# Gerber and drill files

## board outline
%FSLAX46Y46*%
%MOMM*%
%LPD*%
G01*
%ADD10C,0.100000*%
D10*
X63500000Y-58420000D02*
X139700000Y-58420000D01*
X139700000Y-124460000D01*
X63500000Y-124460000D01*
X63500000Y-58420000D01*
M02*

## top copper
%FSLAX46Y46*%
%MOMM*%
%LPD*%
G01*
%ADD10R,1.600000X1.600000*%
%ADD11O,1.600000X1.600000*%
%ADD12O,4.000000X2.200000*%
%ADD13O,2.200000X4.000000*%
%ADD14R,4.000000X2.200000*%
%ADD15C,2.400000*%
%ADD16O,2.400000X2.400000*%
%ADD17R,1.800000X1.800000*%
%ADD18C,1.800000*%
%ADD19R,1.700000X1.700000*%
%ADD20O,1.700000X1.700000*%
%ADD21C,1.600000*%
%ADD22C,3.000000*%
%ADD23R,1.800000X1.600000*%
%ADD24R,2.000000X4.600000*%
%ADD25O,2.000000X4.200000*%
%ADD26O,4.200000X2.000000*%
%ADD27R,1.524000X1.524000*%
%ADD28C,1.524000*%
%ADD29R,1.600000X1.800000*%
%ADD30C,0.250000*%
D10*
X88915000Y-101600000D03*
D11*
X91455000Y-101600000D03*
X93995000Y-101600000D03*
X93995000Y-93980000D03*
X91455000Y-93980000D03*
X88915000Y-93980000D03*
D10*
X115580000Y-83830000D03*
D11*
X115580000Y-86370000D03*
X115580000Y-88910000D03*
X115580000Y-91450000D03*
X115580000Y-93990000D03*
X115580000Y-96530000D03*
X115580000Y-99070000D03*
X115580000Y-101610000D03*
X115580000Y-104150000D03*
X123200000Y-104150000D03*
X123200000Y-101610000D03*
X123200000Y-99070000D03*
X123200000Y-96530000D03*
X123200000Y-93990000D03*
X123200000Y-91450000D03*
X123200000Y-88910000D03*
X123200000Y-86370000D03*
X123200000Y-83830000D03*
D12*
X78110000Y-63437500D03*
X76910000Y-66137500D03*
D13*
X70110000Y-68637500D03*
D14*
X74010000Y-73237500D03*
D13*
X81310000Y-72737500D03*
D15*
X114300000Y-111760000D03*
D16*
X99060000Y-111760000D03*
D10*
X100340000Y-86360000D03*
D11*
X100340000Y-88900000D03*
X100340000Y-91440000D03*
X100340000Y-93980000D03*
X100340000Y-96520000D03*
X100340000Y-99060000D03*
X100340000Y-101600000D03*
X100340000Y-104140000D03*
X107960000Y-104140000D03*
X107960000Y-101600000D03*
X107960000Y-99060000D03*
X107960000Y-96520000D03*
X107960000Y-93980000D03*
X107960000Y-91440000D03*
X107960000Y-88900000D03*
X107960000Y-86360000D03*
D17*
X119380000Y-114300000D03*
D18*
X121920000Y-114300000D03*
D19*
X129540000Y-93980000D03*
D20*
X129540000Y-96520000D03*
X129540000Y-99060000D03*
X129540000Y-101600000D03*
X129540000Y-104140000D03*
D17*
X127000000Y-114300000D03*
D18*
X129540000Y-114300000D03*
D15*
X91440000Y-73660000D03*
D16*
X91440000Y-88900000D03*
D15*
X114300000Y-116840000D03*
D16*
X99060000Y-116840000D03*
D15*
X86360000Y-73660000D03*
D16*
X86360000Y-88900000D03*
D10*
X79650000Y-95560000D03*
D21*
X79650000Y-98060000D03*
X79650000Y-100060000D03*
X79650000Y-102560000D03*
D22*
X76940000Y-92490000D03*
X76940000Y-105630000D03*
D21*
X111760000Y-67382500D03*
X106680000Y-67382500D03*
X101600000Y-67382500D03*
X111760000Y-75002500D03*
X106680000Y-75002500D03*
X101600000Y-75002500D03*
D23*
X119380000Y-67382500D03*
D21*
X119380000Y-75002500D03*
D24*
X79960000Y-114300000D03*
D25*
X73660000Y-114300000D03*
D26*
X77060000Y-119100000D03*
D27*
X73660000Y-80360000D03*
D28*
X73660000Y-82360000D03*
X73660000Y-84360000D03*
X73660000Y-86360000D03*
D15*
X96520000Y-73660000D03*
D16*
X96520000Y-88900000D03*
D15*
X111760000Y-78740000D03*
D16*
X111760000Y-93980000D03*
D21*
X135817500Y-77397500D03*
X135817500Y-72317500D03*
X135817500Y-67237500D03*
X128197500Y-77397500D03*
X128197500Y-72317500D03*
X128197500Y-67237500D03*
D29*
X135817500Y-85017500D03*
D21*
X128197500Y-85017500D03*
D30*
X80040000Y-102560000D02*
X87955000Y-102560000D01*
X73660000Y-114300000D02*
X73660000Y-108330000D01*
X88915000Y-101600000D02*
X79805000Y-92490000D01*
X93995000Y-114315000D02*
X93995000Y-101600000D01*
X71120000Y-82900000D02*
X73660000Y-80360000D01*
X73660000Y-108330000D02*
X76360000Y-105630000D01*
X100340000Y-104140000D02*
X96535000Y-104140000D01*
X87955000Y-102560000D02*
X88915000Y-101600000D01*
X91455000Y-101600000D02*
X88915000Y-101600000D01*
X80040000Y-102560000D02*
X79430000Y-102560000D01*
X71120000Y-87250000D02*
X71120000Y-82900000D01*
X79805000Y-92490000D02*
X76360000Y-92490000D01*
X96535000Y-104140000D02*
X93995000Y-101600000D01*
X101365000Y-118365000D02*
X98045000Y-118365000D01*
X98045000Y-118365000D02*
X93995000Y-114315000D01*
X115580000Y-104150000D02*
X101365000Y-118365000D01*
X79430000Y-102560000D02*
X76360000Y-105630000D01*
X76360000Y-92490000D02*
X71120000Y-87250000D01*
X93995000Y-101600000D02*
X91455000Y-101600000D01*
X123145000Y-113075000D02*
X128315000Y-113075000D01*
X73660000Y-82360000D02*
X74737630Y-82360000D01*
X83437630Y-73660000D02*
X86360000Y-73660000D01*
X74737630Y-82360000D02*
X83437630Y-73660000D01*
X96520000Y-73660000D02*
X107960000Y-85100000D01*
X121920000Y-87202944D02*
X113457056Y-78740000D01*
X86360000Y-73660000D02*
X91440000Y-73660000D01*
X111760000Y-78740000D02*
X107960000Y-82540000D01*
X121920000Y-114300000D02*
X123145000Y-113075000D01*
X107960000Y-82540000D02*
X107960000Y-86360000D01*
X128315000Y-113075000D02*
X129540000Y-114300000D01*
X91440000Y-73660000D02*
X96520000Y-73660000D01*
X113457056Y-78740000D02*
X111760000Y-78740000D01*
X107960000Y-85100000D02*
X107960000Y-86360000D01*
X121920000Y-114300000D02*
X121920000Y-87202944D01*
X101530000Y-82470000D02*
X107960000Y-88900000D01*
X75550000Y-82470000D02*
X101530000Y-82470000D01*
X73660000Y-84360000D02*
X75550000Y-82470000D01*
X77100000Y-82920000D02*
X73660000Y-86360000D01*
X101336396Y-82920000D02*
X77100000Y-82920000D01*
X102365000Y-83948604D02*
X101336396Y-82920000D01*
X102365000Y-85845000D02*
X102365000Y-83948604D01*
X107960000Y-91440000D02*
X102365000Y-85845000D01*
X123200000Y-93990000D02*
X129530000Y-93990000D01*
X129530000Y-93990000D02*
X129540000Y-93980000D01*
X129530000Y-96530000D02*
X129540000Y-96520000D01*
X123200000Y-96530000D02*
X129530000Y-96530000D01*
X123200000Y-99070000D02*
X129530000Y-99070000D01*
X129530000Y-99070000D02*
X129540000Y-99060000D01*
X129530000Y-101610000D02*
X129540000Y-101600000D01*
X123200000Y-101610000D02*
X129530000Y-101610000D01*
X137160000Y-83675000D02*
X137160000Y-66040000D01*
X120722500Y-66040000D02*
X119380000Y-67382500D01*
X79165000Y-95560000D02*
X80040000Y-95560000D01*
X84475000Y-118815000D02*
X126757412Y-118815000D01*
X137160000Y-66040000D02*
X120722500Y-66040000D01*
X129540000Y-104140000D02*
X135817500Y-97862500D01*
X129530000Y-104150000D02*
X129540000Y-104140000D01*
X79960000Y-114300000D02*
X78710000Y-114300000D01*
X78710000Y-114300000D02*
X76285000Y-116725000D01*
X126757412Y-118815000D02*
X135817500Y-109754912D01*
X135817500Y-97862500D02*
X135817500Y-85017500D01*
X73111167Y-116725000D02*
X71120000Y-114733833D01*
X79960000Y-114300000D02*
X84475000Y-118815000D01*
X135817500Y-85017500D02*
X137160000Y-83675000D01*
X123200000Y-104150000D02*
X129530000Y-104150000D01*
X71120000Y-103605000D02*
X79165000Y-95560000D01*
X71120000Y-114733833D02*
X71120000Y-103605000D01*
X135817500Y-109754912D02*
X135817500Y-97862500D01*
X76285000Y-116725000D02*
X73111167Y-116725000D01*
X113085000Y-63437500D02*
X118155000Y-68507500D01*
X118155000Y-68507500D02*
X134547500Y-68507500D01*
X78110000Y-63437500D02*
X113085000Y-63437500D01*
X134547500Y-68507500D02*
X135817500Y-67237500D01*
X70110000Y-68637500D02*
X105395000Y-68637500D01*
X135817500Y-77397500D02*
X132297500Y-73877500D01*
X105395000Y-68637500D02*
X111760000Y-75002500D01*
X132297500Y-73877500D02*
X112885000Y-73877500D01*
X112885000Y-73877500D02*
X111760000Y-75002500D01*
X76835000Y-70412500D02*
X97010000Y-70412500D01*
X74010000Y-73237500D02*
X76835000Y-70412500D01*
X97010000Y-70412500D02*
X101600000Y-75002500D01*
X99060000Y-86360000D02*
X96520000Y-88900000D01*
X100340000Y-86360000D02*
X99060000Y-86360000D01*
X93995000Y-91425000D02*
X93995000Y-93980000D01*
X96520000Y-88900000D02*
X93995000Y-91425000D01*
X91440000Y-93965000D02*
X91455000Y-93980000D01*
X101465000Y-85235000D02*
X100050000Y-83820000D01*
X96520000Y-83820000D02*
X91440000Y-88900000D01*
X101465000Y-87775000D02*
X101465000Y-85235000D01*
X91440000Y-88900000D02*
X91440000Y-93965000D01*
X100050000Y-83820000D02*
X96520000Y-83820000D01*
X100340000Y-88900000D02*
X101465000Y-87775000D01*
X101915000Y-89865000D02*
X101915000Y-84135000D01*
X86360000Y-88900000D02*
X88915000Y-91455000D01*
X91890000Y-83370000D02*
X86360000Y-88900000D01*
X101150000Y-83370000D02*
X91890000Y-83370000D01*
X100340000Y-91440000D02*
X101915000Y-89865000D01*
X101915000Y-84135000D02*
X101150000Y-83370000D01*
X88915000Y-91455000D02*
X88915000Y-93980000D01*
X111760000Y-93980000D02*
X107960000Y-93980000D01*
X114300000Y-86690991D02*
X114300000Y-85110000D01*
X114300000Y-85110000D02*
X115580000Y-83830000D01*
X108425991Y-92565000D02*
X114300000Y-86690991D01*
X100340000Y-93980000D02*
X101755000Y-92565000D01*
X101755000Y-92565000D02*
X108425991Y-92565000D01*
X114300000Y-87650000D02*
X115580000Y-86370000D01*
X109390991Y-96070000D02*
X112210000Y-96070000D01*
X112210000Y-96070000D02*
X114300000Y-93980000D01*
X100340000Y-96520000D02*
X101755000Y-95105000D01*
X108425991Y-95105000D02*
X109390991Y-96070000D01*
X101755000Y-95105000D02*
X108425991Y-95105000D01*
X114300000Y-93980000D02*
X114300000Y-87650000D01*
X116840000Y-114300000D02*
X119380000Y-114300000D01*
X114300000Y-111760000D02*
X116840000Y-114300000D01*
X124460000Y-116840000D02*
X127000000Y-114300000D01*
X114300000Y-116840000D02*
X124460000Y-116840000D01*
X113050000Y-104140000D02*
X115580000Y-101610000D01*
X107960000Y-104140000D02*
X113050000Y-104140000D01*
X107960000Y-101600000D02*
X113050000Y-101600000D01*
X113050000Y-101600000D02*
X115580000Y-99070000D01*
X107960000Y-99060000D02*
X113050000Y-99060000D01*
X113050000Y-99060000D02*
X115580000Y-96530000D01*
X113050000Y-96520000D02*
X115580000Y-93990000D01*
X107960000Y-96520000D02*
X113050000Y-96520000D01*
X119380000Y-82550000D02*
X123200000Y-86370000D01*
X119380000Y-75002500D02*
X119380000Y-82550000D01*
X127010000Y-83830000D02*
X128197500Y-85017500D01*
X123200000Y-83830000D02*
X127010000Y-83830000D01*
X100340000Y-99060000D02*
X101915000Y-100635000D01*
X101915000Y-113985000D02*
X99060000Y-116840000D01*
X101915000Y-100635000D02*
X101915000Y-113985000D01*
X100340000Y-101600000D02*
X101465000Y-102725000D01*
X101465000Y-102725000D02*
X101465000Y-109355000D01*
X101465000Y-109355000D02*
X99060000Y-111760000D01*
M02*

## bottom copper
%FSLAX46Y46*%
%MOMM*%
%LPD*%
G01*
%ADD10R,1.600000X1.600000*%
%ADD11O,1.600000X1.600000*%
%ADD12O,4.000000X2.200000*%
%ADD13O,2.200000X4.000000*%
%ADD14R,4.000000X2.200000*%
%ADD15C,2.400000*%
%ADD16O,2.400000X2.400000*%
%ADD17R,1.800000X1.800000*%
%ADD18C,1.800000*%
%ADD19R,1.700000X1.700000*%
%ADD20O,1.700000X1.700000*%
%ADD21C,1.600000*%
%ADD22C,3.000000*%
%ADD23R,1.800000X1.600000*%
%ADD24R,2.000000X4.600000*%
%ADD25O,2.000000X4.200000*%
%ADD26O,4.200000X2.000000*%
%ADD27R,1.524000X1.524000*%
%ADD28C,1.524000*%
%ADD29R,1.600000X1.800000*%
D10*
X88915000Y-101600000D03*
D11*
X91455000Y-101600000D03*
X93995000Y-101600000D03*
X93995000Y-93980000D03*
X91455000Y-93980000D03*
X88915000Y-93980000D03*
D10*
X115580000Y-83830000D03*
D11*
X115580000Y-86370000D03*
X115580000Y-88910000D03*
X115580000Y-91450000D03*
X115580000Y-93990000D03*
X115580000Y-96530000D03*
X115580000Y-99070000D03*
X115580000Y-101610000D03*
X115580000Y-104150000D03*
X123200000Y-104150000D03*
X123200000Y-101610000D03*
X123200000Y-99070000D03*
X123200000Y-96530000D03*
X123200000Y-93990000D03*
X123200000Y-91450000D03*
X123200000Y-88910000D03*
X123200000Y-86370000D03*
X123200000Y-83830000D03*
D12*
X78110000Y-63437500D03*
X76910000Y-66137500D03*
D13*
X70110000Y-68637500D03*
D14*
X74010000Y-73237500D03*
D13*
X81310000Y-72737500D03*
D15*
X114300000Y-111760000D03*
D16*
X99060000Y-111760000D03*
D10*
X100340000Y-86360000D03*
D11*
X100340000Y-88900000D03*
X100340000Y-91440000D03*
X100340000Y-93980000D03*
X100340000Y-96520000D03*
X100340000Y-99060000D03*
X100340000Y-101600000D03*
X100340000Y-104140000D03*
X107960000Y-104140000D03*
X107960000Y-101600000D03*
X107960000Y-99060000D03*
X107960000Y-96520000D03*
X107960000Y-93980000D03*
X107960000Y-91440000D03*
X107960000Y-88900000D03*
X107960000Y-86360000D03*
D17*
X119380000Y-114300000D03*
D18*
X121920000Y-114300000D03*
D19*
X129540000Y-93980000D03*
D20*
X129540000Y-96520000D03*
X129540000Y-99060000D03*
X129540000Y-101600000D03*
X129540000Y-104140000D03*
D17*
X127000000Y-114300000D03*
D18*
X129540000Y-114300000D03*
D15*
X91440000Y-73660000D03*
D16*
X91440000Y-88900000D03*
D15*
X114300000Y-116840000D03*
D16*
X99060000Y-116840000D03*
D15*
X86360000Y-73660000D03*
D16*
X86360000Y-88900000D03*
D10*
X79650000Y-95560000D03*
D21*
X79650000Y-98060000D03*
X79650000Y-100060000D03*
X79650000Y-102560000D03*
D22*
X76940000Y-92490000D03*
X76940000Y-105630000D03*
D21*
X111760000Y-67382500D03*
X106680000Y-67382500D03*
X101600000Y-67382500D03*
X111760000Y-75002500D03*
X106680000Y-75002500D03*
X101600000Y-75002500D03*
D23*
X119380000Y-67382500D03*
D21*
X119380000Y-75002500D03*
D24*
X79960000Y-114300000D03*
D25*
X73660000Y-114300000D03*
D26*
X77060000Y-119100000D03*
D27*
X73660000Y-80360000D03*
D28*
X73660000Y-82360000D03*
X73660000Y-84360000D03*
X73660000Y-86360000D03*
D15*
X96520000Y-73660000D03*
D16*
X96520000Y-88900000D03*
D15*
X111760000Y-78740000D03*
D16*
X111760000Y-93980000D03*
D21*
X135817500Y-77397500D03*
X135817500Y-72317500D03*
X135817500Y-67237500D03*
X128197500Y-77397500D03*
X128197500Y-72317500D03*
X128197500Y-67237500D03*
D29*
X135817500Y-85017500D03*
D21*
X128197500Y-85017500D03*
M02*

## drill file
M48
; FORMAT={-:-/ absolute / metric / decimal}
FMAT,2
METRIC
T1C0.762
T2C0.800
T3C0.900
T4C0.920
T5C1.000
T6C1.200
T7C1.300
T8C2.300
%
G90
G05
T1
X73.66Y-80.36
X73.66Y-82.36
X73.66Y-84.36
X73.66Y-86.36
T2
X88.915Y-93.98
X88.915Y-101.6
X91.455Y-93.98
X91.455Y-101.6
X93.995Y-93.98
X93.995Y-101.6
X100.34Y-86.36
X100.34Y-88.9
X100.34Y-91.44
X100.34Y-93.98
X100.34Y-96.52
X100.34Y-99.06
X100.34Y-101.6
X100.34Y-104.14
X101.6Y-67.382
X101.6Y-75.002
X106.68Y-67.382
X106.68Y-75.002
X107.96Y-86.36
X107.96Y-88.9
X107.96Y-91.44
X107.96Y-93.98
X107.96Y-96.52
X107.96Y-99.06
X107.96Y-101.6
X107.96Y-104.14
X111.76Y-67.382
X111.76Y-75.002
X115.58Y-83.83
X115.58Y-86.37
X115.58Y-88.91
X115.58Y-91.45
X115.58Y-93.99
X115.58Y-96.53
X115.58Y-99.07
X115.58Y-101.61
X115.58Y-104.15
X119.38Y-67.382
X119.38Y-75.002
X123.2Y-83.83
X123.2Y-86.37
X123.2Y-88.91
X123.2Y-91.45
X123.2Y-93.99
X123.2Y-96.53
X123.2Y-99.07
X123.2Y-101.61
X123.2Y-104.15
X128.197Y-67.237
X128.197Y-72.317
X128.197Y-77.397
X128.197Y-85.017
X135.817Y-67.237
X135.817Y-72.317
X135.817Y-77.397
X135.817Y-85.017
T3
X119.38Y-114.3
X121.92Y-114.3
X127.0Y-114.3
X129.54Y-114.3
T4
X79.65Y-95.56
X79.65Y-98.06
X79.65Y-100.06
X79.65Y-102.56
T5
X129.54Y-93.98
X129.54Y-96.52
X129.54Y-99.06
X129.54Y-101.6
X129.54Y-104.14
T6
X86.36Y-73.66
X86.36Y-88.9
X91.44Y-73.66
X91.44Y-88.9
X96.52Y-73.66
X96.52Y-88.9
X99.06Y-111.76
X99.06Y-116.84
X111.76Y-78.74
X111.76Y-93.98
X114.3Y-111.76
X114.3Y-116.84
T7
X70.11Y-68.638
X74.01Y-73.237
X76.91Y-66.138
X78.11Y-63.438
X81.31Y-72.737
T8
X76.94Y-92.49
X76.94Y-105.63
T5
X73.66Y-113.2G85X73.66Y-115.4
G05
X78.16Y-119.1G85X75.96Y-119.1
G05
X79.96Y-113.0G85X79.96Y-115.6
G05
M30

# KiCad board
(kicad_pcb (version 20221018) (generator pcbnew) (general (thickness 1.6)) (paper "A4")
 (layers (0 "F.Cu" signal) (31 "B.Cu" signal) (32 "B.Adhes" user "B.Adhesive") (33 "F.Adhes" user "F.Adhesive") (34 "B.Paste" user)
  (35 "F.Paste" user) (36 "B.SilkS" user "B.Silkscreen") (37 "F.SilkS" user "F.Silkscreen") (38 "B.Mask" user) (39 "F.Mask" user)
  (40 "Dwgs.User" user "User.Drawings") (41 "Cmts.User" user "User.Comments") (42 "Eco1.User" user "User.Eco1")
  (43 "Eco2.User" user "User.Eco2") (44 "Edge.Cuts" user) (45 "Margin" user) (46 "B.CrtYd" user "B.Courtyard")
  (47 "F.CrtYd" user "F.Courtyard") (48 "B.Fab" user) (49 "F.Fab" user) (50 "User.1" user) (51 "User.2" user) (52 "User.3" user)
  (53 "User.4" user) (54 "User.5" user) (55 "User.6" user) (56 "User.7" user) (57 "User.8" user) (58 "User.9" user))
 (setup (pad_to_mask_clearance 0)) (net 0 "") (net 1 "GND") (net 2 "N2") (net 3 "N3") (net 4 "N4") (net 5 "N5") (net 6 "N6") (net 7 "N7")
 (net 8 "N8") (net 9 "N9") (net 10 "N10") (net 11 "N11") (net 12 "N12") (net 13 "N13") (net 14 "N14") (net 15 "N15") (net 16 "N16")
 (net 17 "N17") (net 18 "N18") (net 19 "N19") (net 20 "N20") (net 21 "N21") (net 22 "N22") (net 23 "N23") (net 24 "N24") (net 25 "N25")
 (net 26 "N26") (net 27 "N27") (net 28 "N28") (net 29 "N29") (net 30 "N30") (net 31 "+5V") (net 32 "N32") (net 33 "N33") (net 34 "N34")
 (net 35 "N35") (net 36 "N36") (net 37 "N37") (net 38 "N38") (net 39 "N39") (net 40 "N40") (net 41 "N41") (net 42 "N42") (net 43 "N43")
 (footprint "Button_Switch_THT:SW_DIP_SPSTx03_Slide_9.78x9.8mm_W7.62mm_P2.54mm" (layer "F.Cu") (at 88.915 101.6 90)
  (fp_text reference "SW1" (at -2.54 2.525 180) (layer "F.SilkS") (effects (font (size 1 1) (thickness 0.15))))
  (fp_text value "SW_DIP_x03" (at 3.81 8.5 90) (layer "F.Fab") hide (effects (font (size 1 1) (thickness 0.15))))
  (pad "1" thru_hole rect (at 0 0 90) (size 1.6 1.6) (drill 0.8) (layers "*.Cu" "*.Mask") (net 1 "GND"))
  (pad "2" thru_hole oval (at 0 2.54 90) (size 1.6 1.6) (drill 0.8) (layers "*.Cu" "*.Mask") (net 1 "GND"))
  (pad "3" thru_hole oval (at 0 5.08 90) (size 1.6 1.6) (drill 0.8) (layers "*.Cu" "*.Mask") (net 1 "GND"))
  (pad "4" thru_hole oval (at 7.62 5.08 90) (size 1.6 1.6) (drill 0.8) (layers "*.Cu" "*.Mask") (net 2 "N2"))
  (pad "5" thru_hole oval (at 7.62 2.54 90) (size 1.6 1.6) (drill 0.8) (layers "*.Cu" "*.Mask") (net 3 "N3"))
  (pad "6" thru_hole oval (at 7.62 0 90) (size 1.6 1.6) (drill 0.8) (layers "*.Cu" "*.Mask") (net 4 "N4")))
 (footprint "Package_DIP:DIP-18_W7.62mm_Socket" (layer "F.Cu") (at 115.58 83.83)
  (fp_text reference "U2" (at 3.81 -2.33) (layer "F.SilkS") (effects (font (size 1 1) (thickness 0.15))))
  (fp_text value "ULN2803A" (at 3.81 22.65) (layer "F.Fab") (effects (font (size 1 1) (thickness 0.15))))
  (pad "1" thru_hole rect (at 0 0) (size 1.6 1.6) (drill 0.8) (layers "*.Cu" "*.Mask") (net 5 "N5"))
  (pad "2" thru_hole oval (at 0 2.54) (size 1.6 1.6) (drill 0.8) (layers "*.Cu" "*.Mask") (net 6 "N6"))
  (pad "3" thru_hole oval (at 0 5.08) (size 1.6 1.6) (drill 0.8) (layers "*.Cu" "*.Mask") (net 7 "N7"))
  (pad "4" thru_hole oval (at 0 7.62) (size 1.6 1.6) (drill 0.8) (layers "*.Cu" "*.Mask") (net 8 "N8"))
  (pad "5" thru_hole oval (at 0 10.16) (size 1.6 1.6) (drill 0.8) (layers "*.Cu" "*.Mask") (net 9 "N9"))
  (pad "6" thru_hole oval (at 0 12.7) (size 1.6 1.6) (drill 0.8) (layers "*.Cu" "*.Mask") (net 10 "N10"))
  (pad "7" thru_hole oval (at 0 15.24) (size 1.6 1.6) (drill 0.8) (layers "*.Cu" "*.Mask") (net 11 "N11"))
  (pad "8" thru_hole oval (at 0 17.78) (size 1.6 1.6) (drill 0.8) (layers "*.Cu" "*.Mask") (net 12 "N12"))
  (pad "9" thru_hole oval (at 0 20.32) (size 1.6 1.6) (drill 0.8) (layers "*.Cu" "*.Mask") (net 1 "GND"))
  (pad "10" thru_hole oval (at 7.62 20.32) (size 1.6 1.6) (drill 0.8) (layers "*.Cu" "*.Mask") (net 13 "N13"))
  (pad "11" thru_hole oval (at 7.62 17.78) (size 1.6 1.6) (drill 0.8) (layers "*.Cu" "*.Mask") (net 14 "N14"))
  (pad "12" thru_hole oval (at 7.62 15.24) (size 1.6 1.6) (drill 0.8) (layers "*.Cu" "*.Mask") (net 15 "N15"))
  (pad "13" thru_hole oval (at 7.62 12.7) (size 1.6 1.6) (drill 0.8) (layers "*.Cu" "*.Mask") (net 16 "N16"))
  (pad "14" thru_hole oval (at 7.62 10.16) (size 1.6 1.6) (drill 0.8) (layers "*.Cu" "*.Mask") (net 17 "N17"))
  (pad "15" thru_hole oval (at 7.62 7.62) (size 1.6 1.6) (drill 0.8) (layers "*.Cu" "*.Mask") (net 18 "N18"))
  (pad "16" thru_hole oval (at 7.62 5.08) (size 1.6 1.6) (drill 0.8) (layers "*.Cu" "*.Mask") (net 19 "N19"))
  (pad "17" thru_hole oval (at 7.62 2.54) (size 1.6 1.6) (drill 0.8) (layers "*.Cu" "*.Mask") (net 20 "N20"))
  (pad "18" thru_hole oval (at 7.62 0) (size 1.6 1.6) (drill 0.8) (layers "*.Cu" "*.Mask") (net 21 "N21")))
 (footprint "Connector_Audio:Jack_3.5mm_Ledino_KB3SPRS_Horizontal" (layer "F.Cu") (at 74.01 73.2375)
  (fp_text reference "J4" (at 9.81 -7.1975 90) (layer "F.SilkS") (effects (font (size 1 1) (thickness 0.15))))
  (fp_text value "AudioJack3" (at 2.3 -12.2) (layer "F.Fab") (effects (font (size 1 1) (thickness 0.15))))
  (pad "R" thru_hole oval (at 4.1 -9.8) (size 4 2.2) (drill 1.3) (layers "*.Cu" "*.Mask") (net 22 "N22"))
  (pad "RN" thru_hole oval (at 2.9 -7.1) (size 4 2.2) (drill 1.3) (layers "*.Cu" "*.Mask"))
  (pad "S" thru_hole oval (at -3.9 -4.6) (size 2.2 4) (drill 1.3) (layers "*.Cu" "*.Mask") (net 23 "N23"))
  (pad "T" thru_hole rect (at 0 0) (size 4 2.2) (drill 1.3) (layers "*.Cu" "*.Mask") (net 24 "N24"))
  (pad "TN" thru_hole oval (at 7.3 -0.5 90) (size 4 2.2) (drill 1.3) (layers "*.Cu" "*.Mask")))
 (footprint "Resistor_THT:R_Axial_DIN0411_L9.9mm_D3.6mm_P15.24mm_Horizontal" (layer "F.Cu") (at 114.3 111.76 180)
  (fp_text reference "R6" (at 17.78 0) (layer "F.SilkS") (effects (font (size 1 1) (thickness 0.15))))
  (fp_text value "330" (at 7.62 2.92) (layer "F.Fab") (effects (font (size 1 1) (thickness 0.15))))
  (pad "1" thru_hole circle (at 0 0 180) (size 2.4 2.4) (drill 1.2) (layers "*.Cu" "*.Mask") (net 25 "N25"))
  (pad "2" thru_hole oval (at 15.24 0 180) (size 2.4 2.4) (drill 1.2) (layers "*.Cu" "*.Mask") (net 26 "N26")))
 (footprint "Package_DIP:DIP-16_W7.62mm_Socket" (layer "F.Cu") (at 100.34 86.36)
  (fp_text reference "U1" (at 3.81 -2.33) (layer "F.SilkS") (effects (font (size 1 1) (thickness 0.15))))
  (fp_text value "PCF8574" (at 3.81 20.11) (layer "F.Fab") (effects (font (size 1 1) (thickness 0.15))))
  (pad "1" thru_hole rect (at 0 0) (size 1.6 1.6) (drill 0.8) (layers "*.Cu" "*.Mask") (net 2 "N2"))
  (pad "2" thru_hole oval (at 0 2.54) (size 1.6 1.6) (drill 0.8) (layers "*.Cu" "*.Mask") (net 3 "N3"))
  (pad "3" thru_hole oval (at 0 5.08) (size 1.6 1.6) (drill 0.8) (layers "*.Cu" "*.Mask") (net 4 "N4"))
  (pad "4" thru_hole oval (at 0 7.62) (size 1.6 1.6) (drill 0.8) (layers "*.Cu" "*.Mask") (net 5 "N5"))
  (pad "5" thru_hole oval (at 0 10.16) (size 1.6 1.6) (drill 0.8) (layers "*.Cu" "*.Mask") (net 6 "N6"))
  (pad "6" thru_hole oval (at 0 12.7) (size 1.6 1.6) (drill 0.8) (layers "*.Cu" "*.Mask") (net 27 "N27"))
  (pad "7" thru_hole oval (at 0 15.24) (size 1.6 1.6) (drill 0.8) (layers "*.Cu" "*.Mask") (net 26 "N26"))
  (pad "8" thru_hole oval (at 0 17.78) (size 1.6 1.6) (drill 0.8) (layers "*.Cu" "*.Mask") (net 1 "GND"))
  (pad "9" thru_hole oval (at 7.62 17.78) (size 1.6 1.6) (drill 0.8) (layers "*.Cu" "*.Mask") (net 12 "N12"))
  (pad "10" thru_hole oval (at 7.62 15.24) (size 1.6 1.6) (drill 0.8) (layers "*.Cu" "*.Mask") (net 11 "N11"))
  (pad "11" thru_hole oval (at 7.62 12.7) (size 1.6 1.6) (drill 0.8) (layers "*.Cu" "*.Mask") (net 10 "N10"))
  (pad "12" thru_hole oval (at 7.62 10.16) (size 1.6 1.6) (drill 0.8) (layers "*.Cu" "*.Mask") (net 9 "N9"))
  (pad "13" thru_hole oval (at 7.62 7.62) (size 1.6 1.6) (drill 0.8) (layers "*.Cu" "*.Mask") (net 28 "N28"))
  (pad "14" thru_hole oval (at 7.62 5.08) (size 1.6 1.6) (drill 0.8) (layers "*.Cu" "*.Mask") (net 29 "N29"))
  (pad "15" thru_hole oval (at 7.62 2.54) (size 1.6 1.6) (drill 0.8) (layers "*.Cu" "*.Mask") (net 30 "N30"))
  (pad "16" thru_hole oval (at 7.62 0) (size 1.6 1.6) (drill 0.8) (layers "*.Cu" "*.Mask") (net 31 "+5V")))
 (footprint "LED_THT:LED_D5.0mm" (layer "F.Cu") (at 119.38 114.3)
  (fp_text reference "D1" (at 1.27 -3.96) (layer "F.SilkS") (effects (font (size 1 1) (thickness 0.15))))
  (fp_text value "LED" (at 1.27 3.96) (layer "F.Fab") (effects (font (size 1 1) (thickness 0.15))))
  (pad "1" thru_hole rect (at 0 0) (size 1.8 1.8) (drill 0.9) (layers "*.Cu" "*.Mask") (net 25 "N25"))
  (pad "2" thru_hole circle (at 2.54 0) (size 1.8 1.8) (drill 0.9) (layers "*.Cu" "*.Mask") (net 31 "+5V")))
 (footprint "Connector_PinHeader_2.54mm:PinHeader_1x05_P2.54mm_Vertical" (layer "F.Cu") (at 129.54 93.98)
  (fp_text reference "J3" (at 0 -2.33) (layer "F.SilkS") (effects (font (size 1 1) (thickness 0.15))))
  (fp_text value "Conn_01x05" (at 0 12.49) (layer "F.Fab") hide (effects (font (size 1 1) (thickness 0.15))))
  (pad "1" thru_hole rect (at 0 0) (size 1.7 1.7) (drill 1) (layers "*.Cu" "*.Mask") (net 17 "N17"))
  (pad "2" thru_hole oval (at 0 2.54) (size 1.7 1.7) (drill 1) (layers "*.Cu" "*.Mask") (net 16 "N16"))
  (pad "3" thru_hole oval (at 0 5.08) (size 1.7 1.7) (drill 1) (layers "*.Cu" "*.Mask") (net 15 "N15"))
  (pad "4" thru_hole oval (at 0 7.62) (size 1.7 1.7) (drill 1) (layers "*.Cu" "*.Mask") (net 14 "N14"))
  (pad "5" thru_hole oval (at 0 10.16) (size 1.7 1.7) (drill 1) (layers "*.Cu" "*.Mask") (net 13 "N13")))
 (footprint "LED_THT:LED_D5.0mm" (layer "F.Cu") (at 127 114.3)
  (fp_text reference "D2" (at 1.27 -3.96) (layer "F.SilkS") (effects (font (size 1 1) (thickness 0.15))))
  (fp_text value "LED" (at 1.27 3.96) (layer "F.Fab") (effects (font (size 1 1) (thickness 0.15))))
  (pad "1" thru_hole rect (at 0 0) (size 1.8 1.8) (drill 0.9) (layers "*.Cu" "*.Mask") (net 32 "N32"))
  (pad "2" thru_hole circle (at 2.54 0) (size 1.8 1.8) (drill 0.9) (layers "*.Cu" "*.Mask") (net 31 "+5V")))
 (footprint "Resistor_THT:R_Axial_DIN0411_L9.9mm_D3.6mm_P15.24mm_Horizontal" (layer "F.Cu") (at 91.44 73.66 -90)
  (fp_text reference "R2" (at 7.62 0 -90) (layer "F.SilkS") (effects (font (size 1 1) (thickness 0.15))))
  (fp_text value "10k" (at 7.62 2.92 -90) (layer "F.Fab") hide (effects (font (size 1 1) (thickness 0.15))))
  (pad "1" thru_hole circle (at 0 0 270) (size 2.4 2.4) (drill 1.2) (layers "*.Cu" "*.Mask") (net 31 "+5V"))
  (pad "2" thru_hole oval (at 15.24 0 270) (size 2.4 2.4) (drill 1.2) (layers "*.Cu" "*.Mask") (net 3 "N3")))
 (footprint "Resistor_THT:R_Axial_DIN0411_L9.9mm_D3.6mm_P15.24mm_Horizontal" (layer "F.Cu") (at 114.3 116.84 180)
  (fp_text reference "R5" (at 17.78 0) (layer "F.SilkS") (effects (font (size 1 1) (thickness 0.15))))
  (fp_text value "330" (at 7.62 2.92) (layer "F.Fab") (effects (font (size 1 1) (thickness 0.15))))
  (pad "1" thru_hole circle (at 0 0 180) (size 2.4 2.4) (drill 1.2) (layers "*.Cu" "*.Mask") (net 32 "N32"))
  (pad "2" thru_hole oval (at 15.24 0 180) (size 2.4 2.4) (drill 1.2) (layers "*.Cu" "*.Mask") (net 27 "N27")))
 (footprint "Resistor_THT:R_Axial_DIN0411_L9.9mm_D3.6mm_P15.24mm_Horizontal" (layer "F.Cu") (at 86.36 73.66 -90)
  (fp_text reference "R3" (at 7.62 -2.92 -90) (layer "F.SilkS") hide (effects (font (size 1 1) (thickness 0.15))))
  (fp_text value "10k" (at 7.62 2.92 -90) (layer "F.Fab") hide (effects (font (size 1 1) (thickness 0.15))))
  (pad "1" thru_hole circle (at 0 0 270) (size 2.4 2.4) (drill 1.2) (layers "*.Cu" "*.Mask") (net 31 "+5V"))
  (pad "2" thru_hole oval (at 15.24 0 270) (size 2.4 2.4) (drill 1.2) (layers "*.Cu" "*.Mask") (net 4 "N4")))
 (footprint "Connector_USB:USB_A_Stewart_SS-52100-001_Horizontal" (layer "F.Cu") (at 79.65 95.56 -90)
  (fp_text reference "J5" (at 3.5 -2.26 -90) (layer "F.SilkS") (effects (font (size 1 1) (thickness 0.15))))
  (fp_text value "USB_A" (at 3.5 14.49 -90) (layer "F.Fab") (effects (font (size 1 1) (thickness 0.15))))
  (pad "1" thru_hole rect (at 0 0 270) (size 1.6 1.6) (drill 0.92) (layers "*.Cu" "*.Mask") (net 13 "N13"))
  (pad "2" thru_hole circle (at 2.5 0 270) (size 1.6 1.6) (drill 0.92) (layers "*.Cu" "*.Mask") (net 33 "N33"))
  (pad "3" thru_hole circle (at 4.5 0 270) (size 1.6 1.6) (drill 0.92) (layers "*.Cu" "*.Mask") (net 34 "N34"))
  (pad "4" thru_hole circle (at 7 0 270) (size 1.6 1.6) (drill 0.92) (layers "*.Cu" "*.Mask") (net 1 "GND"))
  (pad "5" thru_hole circle (at -3.07 2.71 270) (size 3 3) (drill 2.3) (layers "*.Cu" "*.Mask") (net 1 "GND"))
  (pad "5" thru_hole circle (at 10.07 2.71 270) (size 3 3) (drill 2.3) (layers "*.Cu" "*.Mask") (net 1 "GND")))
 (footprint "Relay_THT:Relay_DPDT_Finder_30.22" (layer "F.Cu") (at 119.38 67.3825 180)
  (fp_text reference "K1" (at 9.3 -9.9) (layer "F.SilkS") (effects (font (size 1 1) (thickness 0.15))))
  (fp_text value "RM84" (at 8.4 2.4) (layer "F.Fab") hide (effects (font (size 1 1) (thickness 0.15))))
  (pad "11" thru_hole circle (at 7.62 0 270) (size 1.6 1.6) (drill 0.8) (layers "*.Cu" "*.Mask") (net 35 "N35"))
  (pad "12" thru_hole circle (at 12.7 0 270) (size 1.6 1.6) (drill 0.8) (layers "*.Cu" "*.Mask") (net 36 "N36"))
  (pad "14" thru_hole circle (at 17.78 0 270) (size 1.6 1.6) (drill 0.8) (layers "*.Cu" "*.Mask") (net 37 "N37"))
  (pad "21" thru_hole circle (at 7.62 -7.62 270) (size 1.6 1.6) (drill 0.8) (layers "*.Cu" "*.Mask") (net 23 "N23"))
  (pad "22" thru_hole circle (at 12.7 -7.62 270) (size 1.6 1.6) (drill 0.8) (layers "*.Cu" "*.Mask") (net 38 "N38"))
  (pad "24" thru_hole circle (at 17.78 -7.62) (size 1.6 1.6) (drill 0.8) (layers "*.Cu" "*.Mask") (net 24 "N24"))
  (pad "A1" thru_hole rect (at 0 0 270) (size 1.6 1.8) (drill 0.8) (layers "*.Cu" "*.Mask") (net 13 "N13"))
  (pad "A2" thru_hole circle (at 0 -7.62 270) (size 1.6 1.6) (drill 0.8) (layers "*.Cu" "*.Mask") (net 20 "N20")))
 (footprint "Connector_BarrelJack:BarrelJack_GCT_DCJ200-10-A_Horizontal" (layer "F.Cu") (at 79.96 114.3 -90)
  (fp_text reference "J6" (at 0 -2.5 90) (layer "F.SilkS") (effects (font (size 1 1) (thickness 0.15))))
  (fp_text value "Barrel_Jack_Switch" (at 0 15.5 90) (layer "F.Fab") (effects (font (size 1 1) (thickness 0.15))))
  (pad "1" thru_hole rect (at 0 0 270) (size 4.6 2) (drill oval 3.6 1) (layers "*.Cu" "*.Mask") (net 13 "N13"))
  (pad "2" thru_hole oval (at 0 6.3 270) (size 4.2 2) (drill oval 3.2 1) (layers "*.Cu" "*.Mask") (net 1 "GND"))
  (pad "3" thru_hole oval (at 4.8 2.9 270) (size 2 4.2) (drill oval 1 3.2) (layers "*.Cu" "*.Mask") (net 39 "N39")))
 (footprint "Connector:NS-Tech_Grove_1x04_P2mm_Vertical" (layer "F.Cu") (at 73.66 80.36)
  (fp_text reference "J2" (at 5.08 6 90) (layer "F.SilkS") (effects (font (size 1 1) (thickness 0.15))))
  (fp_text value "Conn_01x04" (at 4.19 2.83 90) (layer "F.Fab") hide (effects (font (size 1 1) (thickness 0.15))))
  (pad "1" thru_hole rect (at 0 0) (size 1.524 1.524) (drill 0.762) (layers "*.Cu" "*.Mask") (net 1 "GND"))
  (pad "2" thru_hole circle (at 0 2) (size 1.524 1.524) (drill 0.762) (layers "*.Cu" "*.Mask") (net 31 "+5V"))
  (pad "3" thru_hole circle (at 0 4) (size 1.524 1.524) (drill 0.762) (layers "*.Cu" "*.Mask") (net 30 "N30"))
  (pad "4" thru_hole circle (at 0 6) (size 1.524 1.524) (drill 0.762) (layers "*.Cu" "*.Mask") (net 29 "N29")))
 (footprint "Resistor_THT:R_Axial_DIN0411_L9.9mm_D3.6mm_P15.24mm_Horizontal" (layer "F.Cu") (at 96.52 73.66 -90)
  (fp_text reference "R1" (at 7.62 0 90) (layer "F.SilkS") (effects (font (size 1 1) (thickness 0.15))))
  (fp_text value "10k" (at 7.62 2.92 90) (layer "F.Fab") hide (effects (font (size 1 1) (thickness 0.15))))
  (pad "1" thru_hole circle (at 0 0 270) (size 2.4 2.4) (drill 1.2) (layers "*.Cu" "*.Mask") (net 31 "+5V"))
  (pad "2" thru_hole oval (at 15.24 0 270) (size 2.4 2.4) (drill 1.2) (layers "*.Cu" "*.Mask") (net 2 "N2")))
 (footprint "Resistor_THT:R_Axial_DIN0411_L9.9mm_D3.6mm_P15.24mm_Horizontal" (layer "F.Cu") (at 111.76 78.74 -90)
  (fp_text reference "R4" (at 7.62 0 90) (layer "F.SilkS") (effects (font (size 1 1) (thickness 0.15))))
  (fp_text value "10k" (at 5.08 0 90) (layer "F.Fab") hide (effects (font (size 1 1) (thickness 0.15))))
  (pad "1" thru_hole circle (at 0 0 270) (size 2.4 2.4) (drill 1.2) (layers "*.Cu" "*.Mask") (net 31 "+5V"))
  (pad "2" thru_hole oval (at 15.24 0 270) (size 2.4 2.4) (drill 1.2) (layers "*.Cu" "*.Mask") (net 28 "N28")))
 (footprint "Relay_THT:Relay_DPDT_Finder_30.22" (layer "F.Cu") (at 135.8175 85.0175 90)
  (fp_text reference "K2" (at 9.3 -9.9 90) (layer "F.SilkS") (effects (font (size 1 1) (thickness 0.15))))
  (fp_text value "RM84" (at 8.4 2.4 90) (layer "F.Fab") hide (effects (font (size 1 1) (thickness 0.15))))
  (pad "11" thru_hole circle (at 7.62 0 180) (size 1.6 1.6) (drill 0.8) (layers "*.Cu" "*.Mask") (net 23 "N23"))
  (pad "12" thru_hole circle (at 12.7 0 180) (size 1.6 1.6) (drill 0.8) (layers "*.Cu" "*.Mask") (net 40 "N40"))
  (pad "14" thru_hole circle (at 17.78 0 180) (size 1.6 1.6) (drill 0.8) (layers "*.Cu" "*.Mask") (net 22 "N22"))
  (pad "21" thru_hole circle (at 7.62 -7.62 180) (size 1.6 1.6) (drill 0.8) (layers "*.Cu" "*.Mask") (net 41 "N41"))
  (pad "22" thru_hole circle (at 12.7 -7.62 180) (size 1.6 1.6) (drill 0.8) (layers "*.Cu" "*.Mask") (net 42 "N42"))
  (pad "24" thru_hole circle (at 17.78 -7.62 270) (size 1.6 1.6) (drill 0.8) (layers "*.Cu" "*.Mask") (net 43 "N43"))
  (pad "A1" thru_hole rect (at 0 0 180) (size 1.6 1.8) (drill 0.8) (layers "*.Cu" "*.Mask") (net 13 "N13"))
  (pad "A2" thru_hole circle (at 0 -7.62 180) (size 1.6 1.6) (drill 0.8) (layers "*.Cu" "*.Mask") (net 21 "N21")))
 (gr_rect (start 63.5 58.42) (end 139.7 124.46) (stroke (width 0.1) (type default)) (fill none) (layer "Edge.Cuts"))
 (segment (start 80.04 102.56) (end 87.955 102.56) (width 0.25) (layer "F.Cu") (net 1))
 (segment (start 73.66 114.3) (end 73.66 108.33) (width 0.25) (layer "F.Cu") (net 1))
 (segment (start 88.915 101.6) (end 79.805 92.49) (width 0.25) (layer "F.Cu") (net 1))
 (segment (start 93.995 114.315) (end 93.995 101.6) (width 0.25) (layer "F.Cu") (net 1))
 (segment (start 71.12 82.9) (end 73.66 80.36) (width 0.25) (layer "F.Cu") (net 1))
 (segment (start 73.66 108.33) (end 76.36 105.63) (width 0.25) (layer "F.Cu") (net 1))
 (segment (start 100.34 104.14) (end 96.535 104.14) (width 0.25) (layer "F.Cu") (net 1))
 (segment (start 87.955 102.56) (end 88.915 101.6) (width 0.25) (layer "F.Cu") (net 1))
 (segment (start 91.455 101.6) (end 88.915 101.6) (width 0.25) (layer "F.Cu") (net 1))
 (segment (start 80.04 102.56) (end 79.43 102.56) (width 0.25) (layer "F.Cu") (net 1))
 (segment (start 71.12 87.25) (end 71.12 82.9) (width 0.25) (layer "F.Cu") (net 1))
 (segment (start 79.805 92.49) (end 76.36 92.49) (width 0.25) (layer "F.Cu") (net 1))
 (segment (start 96.535 104.14) (end 93.995 101.6) (width 0.25) (layer "F.Cu") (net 1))
 (segment (start 101.365 118.365) (end 98.045 118.365) (width 0.25) (layer "F.Cu") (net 1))
 (segment (start 98.045 118.365) (end 93.995 114.315) (width 0.25) (layer "F.Cu") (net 1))
 (segment (start 115.58 104.15) (end 101.365 118.365) (width 0.25) (layer "F.Cu") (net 1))
 (segment (start 79.43 102.56) (end 76.36 105.63) (width 0.25) (layer "F.Cu") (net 1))
 (segment (start 76.36 92.49) (end 71.12 87.25) (width 0.25) (layer "F.Cu") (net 1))
 (segment (start 93.995 101.6) (end 91.455 101.6) (width 0.25) (layer "F.Cu") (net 1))
 (segment (start 123.145 113.075) (end 128.315 113.075) (width 0.25) (layer "F.Cu") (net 31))
 (segment (start 73.66 82.36) (end 74.73763 82.36) (width 0.25) (layer "F.Cu") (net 31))
 (segment (start 83.43763 73.66) (end 86.36 73.66) (width 0.25) (layer "F.Cu") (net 31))
 (segment (start 74.73763 82.36) (end 83.43763 73.66) (width 0.25) (layer "F.Cu") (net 31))
 (segment (start 96.52 73.66) (end 107.96 85.1) (width 0.25) (layer "F.Cu") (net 31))
 (segment (start 121.92 87.202944) (end 113.457056 78.74) (width 0.25) (layer "F.Cu") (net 31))
 (segment (start 86.36 73.66) (end 91.44 73.66) (width 0.25) (layer "F.Cu") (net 31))
 (segment (start 111.76 78.74) (end 107.96 82.54) (width 0.25) (layer "F.Cu") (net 31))
 (segment (start 121.92 114.3) (end 123.145 113.075) (width 0.25) (layer "F.Cu") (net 31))
 (segment (start 107.96 82.54) (end 107.96 86.36) (width 0.25) (layer "F.Cu") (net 31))
 (segment (start 128.315 113.075) (end 129.54 114.3) (width 0.25) (layer "F.Cu") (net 31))
 (segment (start 91.44 73.66) (end 96.52 73.66) (width 0.25) (layer "F.Cu") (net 31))
 (segment (start 113.457056 78.74) (end 111.76 78.74) (width 0.25) (layer "F.Cu") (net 31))
 (segment (start 107.96 85.1) (end 107.96 86.36) (width 0.25) (layer "F.Cu") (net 31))
 (segment (start 121.92 114.3) (end 121.92 87.202944) (width 0.25) (layer "F.Cu") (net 31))
 (segment (start 101.53 82.47) (end 107.96 88.9) (width 0.25) (layer "F.Cu") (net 30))
 (segment (start 75.55 82.47) (end 101.53 82.47) (width 0.25) (layer "F.Cu") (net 30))
 (segment (start 73.66 84.36) (end 75.55 82.47) (width 0.25) (layer "F.Cu") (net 30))
 (segment (start 77.1 82.92) (end 73.66 86.36) (width 0.25) (layer "F.Cu") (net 29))
 (segment (start 101.336396 82.92) (end 77.1 82.92) (width 0.25) (layer "F.Cu") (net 29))
 (segment (start 102.365 83.948604) (end 101.336396 82.92) (width 0.25) (layer "F.Cu") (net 29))
 (segment (start 102.365 85.845) (end 102.365 83.948604) (width 0.25) (layer "F.Cu") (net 29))
 (segment (start 107.96 91.44) (end 102.365 85.845) (width 0.25) (layer "F.Cu") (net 29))
 (segment (start 123.2 93.99) (end 129.53 93.99) (width 0.25) (layer "F.Cu") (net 17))
 (segment (start 129.53 93.99) (end 129.54 93.98) (width 0.25) (layer "F.Cu") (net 17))
 (segment (start 129.53 96.53) (end 129.54 96.52) (width 0.25) (layer "F.Cu") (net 16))
 (segment (start 123.2 96.53) (end 129.53 96.53) (width 0.25) (layer "F.Cu") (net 16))
 (segment (start 123.2 99.07) (end 129.53 99.07) (width 0.25) (layer "F.Cu") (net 15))
 (segment (start 129.53 99.07) (end 129.54 99.06) (width 0.25) (layer "F.Cu") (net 15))
 (segment (start 129.53 101.61) (end 129.54 101.6) (width 0.25) (layer "F.Cu") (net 14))
 (segment (start 123.2 101.61) (end 129.53 101.61) (width 0.25) (layer "F.Cu") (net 14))
 (segment (start 137.16 83.675) (end 137.16 66.04) (width 0.25) (layer "F.Cu") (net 13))
 (segment (start 120.7225 66.04) (end 119.38 67.3825) (width 0.25) (layer "F.Cu") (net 13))
 (segment (start 79.165 95.56) (end 80.04 95.56) (width 0.25) (layer "F.Cu") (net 13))
 (segment (start 84.475 118.815) (end 126.757412 118.815) (width 0.25) (layer "F.Cu") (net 13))
 (segment (start 137.16 66.04) (end 120.7225 66.04) (width 0.25) (layer "F.Cu") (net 13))
 (segment (start 129.54 104.14) (end 135.8175 97.8625) (width 0.25) (layer "F.Cu") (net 13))
 (segment (start 129.53 104.15) (end 129.54 104.14) (width 0.25) (layer "F.Cu") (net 13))
 (segment (start 79.96 114.3) (end 78.71 114.3) (width 0.25) (layer "F.Cu") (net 13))
 (segment (start 78.71 114.3) (end 76.285 116.725) (width 0.25) (layer "F.Cu") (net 13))
 (segment (start 126.757412 118.815) (end 135.8175 109.754912) (width 0.25) (layer "F.Cu") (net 13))
 (segment (start 135.8175 97.8625) (end 135.8175 85.0175) (width 0.25) (layer "F.Cu") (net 13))
 (segment (start 73.111167 116.725) (end 71.12 114.733833) (width 0.25) (layer "F.Cu") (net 13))
 (segment (start 79.96 114.3) (end 84.475 118.815) (width 0.25) (layer "F.Cu") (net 13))
 (segment (start 135.8175 85.0175) (end 137.16 83.675) (width 0.25) (layer "F.Cu") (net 13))
 (segment (start 123.2 104.15) (end 129.53 104.15) (width 0.25) (layer "F.Cu") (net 13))
 (segment (start 71.12 103.605) (end 79.165 95.56) (width 0.25) (layer "F.Cu") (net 13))
 (segment (start 71.12 114.733833) (end 71.12 103.605) (width 0.25) (layer "F.Cu") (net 13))
 (segment (start 135.8175 109.754912) (end 135.8175 97.8625) (width 0.25) (layer "F.Cu") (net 13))
 (segment (start 76.285 116.725) (end 73.111167 116.725) (width 0.25) (layer "F.Cu") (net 13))
 (segment (start 113.085 63.4375) (end 118.155 68.5075) (width 0.25) (layer "F.Cu") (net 22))
 (segment (start 118.155 68.5075) (end 134.5475 68.5075) (width 0.25) (layer "F.Cu") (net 22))
 (segment (start 78.11 63.4375) (end 113.085 63.4375) (width 0.25) (layer "F.Cu") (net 22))
 (segment (start 134.5475 68.5075) (end 135.8175 67.2375) (width 0.25) (layer "F.Cu") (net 22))
 (segment (start 70.11 68.6375) (end 105.395 68.6375) (width 0.25) (layer "F.Cu") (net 23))
 (segment (start 135.8175 77.3975) (end 132.2975 73.8775) (width 0.25) (layer "F.Cu") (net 23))
 (segment (start 105.395 68.6375) (end 111.76 75.0025) (width 0.25) (layer "F.Cu") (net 23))
 (segment (start 132.2975 73.8775) (end 112.885 73.8775) (width 0.25) (layer "F.Cu") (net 23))
 (segment (start 112.885 73.8775) (end 111.76 75.0025) (width 0.25) (layer "F.Cu") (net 23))
 (segment (start 76.835 70.4125) (end 97.01 70.4125) (width 0.25) (layer "F.Cu") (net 24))
 (segment (start 74.01 73.2375) (end 76.835 70.4125) (width 0.25) (layer "F.Cu") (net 24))
 (segment (start 97.01 70.4125) (end 101.6 75.0025) (width 0.25) (layer "F.Cu") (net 24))
 (segment (start 99.06 86.36) (end 96.52 88.9) (width 0.25) (layer "F.Cu") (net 2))
 (segment (start 100.34 86.36) (end 99.06 86.36) (width 0.25) (layer "F.Cu") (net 2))
 (segment (start 93.995 91.425) (end 93.995 93.98) (width 0.25) (layer "F.Cu") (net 2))
 (segment (start 96.52 88.9) (end 93.995 91.425) (width 0.25) (layer "F.Cu") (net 2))
 (segment (start 91.44 93.965) (end 91.455 93.98) (width 0.25) (layer "F.Cu") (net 3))
 (segment (start 101.465 85.235) (end 100.05 83.82) (width 0.25) (layer "F.Cu") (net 3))
 (segment (start 96.52 83.82) (end 91.44 88.9) (width 0.25) (layer "F.Cu") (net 3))
 (segment (start 101.465 87.775) (end 101.465 85.235) (width 0.25) (layer "F.Cu") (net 3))
 (segment (start 91.44 88.9) (end 91.44 93.965) (width 0.25) (layer "F.Cu") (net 3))
 (segment (start 100.05 83.82) (end 96.52 83.82) (width 0.25) (layer "F.Cu") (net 3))
 (segment (start 100.34 88.9) (end 101.465 87.775) (width 0.25) (layer "F.Cu") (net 3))
 (segment (start 101.915 89.865) (end 101.915 84.135) (width 0.25) (layer "F.Cu") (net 4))
 (segment (start 86.36 88.9) (end 88.915 91.455) (width 0.25) (layer "F.Cu") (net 4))
 (segment (start 91.89 83.37) (end 86.36 88.9) (width 0.25) (layer "F.Cu") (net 4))
 (segment (start 101.15 83.37) (end 91.89 83.37) (width 0.25) (layer "F.Cu") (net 4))
 (segment (start 100.34 91.44) (end 101.915 89.865) (width 0.25) (layer "F.Cu") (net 4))
 (segment (start 101.915 84.135) (end 101.15 83.37) (width 0.25) (layer "F.Cu") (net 4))
 (segment (start 88.915 91.455) (end 88.915 93.98) (width 0.25) (layer "F.Cu") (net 4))
 (segment (start 111.76 93.98) (end 107.96 93.98) (width 0.25) (layer "F.Cu") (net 28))
 (segment (start 114.3 86.690991) (end 114.3 85.11) (width 0.25) (layer "F.Cu") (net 5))
 (segment (start 114.3 85.11) (end 115.58 83.83) (width 0.25) (layer "F.Cu") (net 5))
 (segment (start 108.425991 92.565) (end 114.3 86.690991) (width 0.25) (layer "F.Cu") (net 5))
 (segment (start 100.34 93.98) (end 101.755 92.565) (width 0.25) (layer "F.Cu") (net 5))
 (segment (start 101.755 92.565) (end 108.425991 92.565) (width 0.25) (layer "F.Cu") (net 5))
 (segment (start 114.3 87.65) (end 115.58 86.37) (width 0.25) (layer "F.Cu") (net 6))
 (segment (start 109.390991 96.07) (end 112.21 96.07) (width 0.25) (layer "F.Cu") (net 6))
 (segment (start 112.21 96.07) (end 114.3 93.98) (width 0.25) (layer "F.Cu") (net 6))
 (segment (start 100.34 96.52) (end 101.755 95.105) (width 0.25) (layer "F.Cu") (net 6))
 (segment (start 108.425991 95.105) (end 109.390991 96.07) (width 0.25) (layer "F.Cu") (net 6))
 (segment (start 101.755 95.105) (end 108.425991 95.105) (width 0.25) (layer "F.Cu") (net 6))
 (segment (start 114.3 93.98) (end 114.3 87.65) (width 0.25) (layer "F.Cu") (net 6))
 (segment (start 116.84 114.3) (end 119.38 114.3) (width 0.25) (layer "F.Cu") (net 25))
 (segment (start 114.3 111.76) (end 116.84 114.3) (width 0.25) (layer "F.Cu") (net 25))
 (segment (start 124.46 116.84) (end 127 114.3) (width 0.25) (layer "F.Cu") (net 32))
 (segment (start 114.3 116.84) (end 124.46 116.84) (width 0.25) (layer "F.Cu") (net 32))
 (segment (start 113.05 104.14) (end 115.58 101.61) (width 0.25) (layer "F.Cu") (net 12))
 (segment (start 107.96 104.14) (end 113.05 104.14) (width 0.25) (layer "F.Cu") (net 12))
 (segment (start 107.96 101.6) (end 113.05 101.6) (width 0.25) (layer "F.Cu") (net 11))
 (segment (start 113.05 101.6) (end 115.58 99.07) (width 0.25) (layer "F.Cu") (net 11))
 (segment (start 107.96 99.06) (end 113.05 99.06) (width 0.25) (layer "F.Cu") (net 10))
 (segment (start 113.05 99.06) (end 115.58 96.53) (width 0.25) (layer "F.Cu") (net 10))
 (segment (start 113.05 96.52) (end 115.58 93.99) (width 0.25) (layer "F.Cu") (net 9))
 (segment (start 107.96 96.52) (end 113.05 96.52) (width 0.25) (layer "F.Cu") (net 9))
 (segment (start 119.38 82.55) (end 123.2 86.37) (width 0.25) (layer "F.Cu") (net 20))
 (segment (start 119.38 75.0025) (end 119.38 82.55) (width 0.25) (layer "F.Cu") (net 20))
 (segment (start 127.01 83.83) (end 128.1975 85.0175) (width 0.25) (layer "F.Cu") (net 21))
 (segment (start 123.2 83.83) (end 127.01 83.83) (width 0.25) (layer "F.Cu") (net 21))
 (segment (start 100.34 99.06) (end 101.915 100.635) (width 0.25) (layer "F.Cu") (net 27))
 (segment (start 101.915 113.985) (end 99.06 116.84) (width 0.25) (layer "F.Cu") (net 27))
 (segment (start 101.915 100.635) (end 101.915 113.985) (width 0.25) (layer "F.Cu") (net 27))
 (segment (start 100.34 101.6) (end 101.465 102.725) (width 0.25) (layer "F.Cu") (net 26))
 (segment (start 101.465 102.725) (end 101.465 109.355) (width 0.25) (layer "F.Cu") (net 26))
 (segment (start 101.465 109.355) (end 99.06 111.76) (width 0.25) (layer "F.Cu") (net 26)))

